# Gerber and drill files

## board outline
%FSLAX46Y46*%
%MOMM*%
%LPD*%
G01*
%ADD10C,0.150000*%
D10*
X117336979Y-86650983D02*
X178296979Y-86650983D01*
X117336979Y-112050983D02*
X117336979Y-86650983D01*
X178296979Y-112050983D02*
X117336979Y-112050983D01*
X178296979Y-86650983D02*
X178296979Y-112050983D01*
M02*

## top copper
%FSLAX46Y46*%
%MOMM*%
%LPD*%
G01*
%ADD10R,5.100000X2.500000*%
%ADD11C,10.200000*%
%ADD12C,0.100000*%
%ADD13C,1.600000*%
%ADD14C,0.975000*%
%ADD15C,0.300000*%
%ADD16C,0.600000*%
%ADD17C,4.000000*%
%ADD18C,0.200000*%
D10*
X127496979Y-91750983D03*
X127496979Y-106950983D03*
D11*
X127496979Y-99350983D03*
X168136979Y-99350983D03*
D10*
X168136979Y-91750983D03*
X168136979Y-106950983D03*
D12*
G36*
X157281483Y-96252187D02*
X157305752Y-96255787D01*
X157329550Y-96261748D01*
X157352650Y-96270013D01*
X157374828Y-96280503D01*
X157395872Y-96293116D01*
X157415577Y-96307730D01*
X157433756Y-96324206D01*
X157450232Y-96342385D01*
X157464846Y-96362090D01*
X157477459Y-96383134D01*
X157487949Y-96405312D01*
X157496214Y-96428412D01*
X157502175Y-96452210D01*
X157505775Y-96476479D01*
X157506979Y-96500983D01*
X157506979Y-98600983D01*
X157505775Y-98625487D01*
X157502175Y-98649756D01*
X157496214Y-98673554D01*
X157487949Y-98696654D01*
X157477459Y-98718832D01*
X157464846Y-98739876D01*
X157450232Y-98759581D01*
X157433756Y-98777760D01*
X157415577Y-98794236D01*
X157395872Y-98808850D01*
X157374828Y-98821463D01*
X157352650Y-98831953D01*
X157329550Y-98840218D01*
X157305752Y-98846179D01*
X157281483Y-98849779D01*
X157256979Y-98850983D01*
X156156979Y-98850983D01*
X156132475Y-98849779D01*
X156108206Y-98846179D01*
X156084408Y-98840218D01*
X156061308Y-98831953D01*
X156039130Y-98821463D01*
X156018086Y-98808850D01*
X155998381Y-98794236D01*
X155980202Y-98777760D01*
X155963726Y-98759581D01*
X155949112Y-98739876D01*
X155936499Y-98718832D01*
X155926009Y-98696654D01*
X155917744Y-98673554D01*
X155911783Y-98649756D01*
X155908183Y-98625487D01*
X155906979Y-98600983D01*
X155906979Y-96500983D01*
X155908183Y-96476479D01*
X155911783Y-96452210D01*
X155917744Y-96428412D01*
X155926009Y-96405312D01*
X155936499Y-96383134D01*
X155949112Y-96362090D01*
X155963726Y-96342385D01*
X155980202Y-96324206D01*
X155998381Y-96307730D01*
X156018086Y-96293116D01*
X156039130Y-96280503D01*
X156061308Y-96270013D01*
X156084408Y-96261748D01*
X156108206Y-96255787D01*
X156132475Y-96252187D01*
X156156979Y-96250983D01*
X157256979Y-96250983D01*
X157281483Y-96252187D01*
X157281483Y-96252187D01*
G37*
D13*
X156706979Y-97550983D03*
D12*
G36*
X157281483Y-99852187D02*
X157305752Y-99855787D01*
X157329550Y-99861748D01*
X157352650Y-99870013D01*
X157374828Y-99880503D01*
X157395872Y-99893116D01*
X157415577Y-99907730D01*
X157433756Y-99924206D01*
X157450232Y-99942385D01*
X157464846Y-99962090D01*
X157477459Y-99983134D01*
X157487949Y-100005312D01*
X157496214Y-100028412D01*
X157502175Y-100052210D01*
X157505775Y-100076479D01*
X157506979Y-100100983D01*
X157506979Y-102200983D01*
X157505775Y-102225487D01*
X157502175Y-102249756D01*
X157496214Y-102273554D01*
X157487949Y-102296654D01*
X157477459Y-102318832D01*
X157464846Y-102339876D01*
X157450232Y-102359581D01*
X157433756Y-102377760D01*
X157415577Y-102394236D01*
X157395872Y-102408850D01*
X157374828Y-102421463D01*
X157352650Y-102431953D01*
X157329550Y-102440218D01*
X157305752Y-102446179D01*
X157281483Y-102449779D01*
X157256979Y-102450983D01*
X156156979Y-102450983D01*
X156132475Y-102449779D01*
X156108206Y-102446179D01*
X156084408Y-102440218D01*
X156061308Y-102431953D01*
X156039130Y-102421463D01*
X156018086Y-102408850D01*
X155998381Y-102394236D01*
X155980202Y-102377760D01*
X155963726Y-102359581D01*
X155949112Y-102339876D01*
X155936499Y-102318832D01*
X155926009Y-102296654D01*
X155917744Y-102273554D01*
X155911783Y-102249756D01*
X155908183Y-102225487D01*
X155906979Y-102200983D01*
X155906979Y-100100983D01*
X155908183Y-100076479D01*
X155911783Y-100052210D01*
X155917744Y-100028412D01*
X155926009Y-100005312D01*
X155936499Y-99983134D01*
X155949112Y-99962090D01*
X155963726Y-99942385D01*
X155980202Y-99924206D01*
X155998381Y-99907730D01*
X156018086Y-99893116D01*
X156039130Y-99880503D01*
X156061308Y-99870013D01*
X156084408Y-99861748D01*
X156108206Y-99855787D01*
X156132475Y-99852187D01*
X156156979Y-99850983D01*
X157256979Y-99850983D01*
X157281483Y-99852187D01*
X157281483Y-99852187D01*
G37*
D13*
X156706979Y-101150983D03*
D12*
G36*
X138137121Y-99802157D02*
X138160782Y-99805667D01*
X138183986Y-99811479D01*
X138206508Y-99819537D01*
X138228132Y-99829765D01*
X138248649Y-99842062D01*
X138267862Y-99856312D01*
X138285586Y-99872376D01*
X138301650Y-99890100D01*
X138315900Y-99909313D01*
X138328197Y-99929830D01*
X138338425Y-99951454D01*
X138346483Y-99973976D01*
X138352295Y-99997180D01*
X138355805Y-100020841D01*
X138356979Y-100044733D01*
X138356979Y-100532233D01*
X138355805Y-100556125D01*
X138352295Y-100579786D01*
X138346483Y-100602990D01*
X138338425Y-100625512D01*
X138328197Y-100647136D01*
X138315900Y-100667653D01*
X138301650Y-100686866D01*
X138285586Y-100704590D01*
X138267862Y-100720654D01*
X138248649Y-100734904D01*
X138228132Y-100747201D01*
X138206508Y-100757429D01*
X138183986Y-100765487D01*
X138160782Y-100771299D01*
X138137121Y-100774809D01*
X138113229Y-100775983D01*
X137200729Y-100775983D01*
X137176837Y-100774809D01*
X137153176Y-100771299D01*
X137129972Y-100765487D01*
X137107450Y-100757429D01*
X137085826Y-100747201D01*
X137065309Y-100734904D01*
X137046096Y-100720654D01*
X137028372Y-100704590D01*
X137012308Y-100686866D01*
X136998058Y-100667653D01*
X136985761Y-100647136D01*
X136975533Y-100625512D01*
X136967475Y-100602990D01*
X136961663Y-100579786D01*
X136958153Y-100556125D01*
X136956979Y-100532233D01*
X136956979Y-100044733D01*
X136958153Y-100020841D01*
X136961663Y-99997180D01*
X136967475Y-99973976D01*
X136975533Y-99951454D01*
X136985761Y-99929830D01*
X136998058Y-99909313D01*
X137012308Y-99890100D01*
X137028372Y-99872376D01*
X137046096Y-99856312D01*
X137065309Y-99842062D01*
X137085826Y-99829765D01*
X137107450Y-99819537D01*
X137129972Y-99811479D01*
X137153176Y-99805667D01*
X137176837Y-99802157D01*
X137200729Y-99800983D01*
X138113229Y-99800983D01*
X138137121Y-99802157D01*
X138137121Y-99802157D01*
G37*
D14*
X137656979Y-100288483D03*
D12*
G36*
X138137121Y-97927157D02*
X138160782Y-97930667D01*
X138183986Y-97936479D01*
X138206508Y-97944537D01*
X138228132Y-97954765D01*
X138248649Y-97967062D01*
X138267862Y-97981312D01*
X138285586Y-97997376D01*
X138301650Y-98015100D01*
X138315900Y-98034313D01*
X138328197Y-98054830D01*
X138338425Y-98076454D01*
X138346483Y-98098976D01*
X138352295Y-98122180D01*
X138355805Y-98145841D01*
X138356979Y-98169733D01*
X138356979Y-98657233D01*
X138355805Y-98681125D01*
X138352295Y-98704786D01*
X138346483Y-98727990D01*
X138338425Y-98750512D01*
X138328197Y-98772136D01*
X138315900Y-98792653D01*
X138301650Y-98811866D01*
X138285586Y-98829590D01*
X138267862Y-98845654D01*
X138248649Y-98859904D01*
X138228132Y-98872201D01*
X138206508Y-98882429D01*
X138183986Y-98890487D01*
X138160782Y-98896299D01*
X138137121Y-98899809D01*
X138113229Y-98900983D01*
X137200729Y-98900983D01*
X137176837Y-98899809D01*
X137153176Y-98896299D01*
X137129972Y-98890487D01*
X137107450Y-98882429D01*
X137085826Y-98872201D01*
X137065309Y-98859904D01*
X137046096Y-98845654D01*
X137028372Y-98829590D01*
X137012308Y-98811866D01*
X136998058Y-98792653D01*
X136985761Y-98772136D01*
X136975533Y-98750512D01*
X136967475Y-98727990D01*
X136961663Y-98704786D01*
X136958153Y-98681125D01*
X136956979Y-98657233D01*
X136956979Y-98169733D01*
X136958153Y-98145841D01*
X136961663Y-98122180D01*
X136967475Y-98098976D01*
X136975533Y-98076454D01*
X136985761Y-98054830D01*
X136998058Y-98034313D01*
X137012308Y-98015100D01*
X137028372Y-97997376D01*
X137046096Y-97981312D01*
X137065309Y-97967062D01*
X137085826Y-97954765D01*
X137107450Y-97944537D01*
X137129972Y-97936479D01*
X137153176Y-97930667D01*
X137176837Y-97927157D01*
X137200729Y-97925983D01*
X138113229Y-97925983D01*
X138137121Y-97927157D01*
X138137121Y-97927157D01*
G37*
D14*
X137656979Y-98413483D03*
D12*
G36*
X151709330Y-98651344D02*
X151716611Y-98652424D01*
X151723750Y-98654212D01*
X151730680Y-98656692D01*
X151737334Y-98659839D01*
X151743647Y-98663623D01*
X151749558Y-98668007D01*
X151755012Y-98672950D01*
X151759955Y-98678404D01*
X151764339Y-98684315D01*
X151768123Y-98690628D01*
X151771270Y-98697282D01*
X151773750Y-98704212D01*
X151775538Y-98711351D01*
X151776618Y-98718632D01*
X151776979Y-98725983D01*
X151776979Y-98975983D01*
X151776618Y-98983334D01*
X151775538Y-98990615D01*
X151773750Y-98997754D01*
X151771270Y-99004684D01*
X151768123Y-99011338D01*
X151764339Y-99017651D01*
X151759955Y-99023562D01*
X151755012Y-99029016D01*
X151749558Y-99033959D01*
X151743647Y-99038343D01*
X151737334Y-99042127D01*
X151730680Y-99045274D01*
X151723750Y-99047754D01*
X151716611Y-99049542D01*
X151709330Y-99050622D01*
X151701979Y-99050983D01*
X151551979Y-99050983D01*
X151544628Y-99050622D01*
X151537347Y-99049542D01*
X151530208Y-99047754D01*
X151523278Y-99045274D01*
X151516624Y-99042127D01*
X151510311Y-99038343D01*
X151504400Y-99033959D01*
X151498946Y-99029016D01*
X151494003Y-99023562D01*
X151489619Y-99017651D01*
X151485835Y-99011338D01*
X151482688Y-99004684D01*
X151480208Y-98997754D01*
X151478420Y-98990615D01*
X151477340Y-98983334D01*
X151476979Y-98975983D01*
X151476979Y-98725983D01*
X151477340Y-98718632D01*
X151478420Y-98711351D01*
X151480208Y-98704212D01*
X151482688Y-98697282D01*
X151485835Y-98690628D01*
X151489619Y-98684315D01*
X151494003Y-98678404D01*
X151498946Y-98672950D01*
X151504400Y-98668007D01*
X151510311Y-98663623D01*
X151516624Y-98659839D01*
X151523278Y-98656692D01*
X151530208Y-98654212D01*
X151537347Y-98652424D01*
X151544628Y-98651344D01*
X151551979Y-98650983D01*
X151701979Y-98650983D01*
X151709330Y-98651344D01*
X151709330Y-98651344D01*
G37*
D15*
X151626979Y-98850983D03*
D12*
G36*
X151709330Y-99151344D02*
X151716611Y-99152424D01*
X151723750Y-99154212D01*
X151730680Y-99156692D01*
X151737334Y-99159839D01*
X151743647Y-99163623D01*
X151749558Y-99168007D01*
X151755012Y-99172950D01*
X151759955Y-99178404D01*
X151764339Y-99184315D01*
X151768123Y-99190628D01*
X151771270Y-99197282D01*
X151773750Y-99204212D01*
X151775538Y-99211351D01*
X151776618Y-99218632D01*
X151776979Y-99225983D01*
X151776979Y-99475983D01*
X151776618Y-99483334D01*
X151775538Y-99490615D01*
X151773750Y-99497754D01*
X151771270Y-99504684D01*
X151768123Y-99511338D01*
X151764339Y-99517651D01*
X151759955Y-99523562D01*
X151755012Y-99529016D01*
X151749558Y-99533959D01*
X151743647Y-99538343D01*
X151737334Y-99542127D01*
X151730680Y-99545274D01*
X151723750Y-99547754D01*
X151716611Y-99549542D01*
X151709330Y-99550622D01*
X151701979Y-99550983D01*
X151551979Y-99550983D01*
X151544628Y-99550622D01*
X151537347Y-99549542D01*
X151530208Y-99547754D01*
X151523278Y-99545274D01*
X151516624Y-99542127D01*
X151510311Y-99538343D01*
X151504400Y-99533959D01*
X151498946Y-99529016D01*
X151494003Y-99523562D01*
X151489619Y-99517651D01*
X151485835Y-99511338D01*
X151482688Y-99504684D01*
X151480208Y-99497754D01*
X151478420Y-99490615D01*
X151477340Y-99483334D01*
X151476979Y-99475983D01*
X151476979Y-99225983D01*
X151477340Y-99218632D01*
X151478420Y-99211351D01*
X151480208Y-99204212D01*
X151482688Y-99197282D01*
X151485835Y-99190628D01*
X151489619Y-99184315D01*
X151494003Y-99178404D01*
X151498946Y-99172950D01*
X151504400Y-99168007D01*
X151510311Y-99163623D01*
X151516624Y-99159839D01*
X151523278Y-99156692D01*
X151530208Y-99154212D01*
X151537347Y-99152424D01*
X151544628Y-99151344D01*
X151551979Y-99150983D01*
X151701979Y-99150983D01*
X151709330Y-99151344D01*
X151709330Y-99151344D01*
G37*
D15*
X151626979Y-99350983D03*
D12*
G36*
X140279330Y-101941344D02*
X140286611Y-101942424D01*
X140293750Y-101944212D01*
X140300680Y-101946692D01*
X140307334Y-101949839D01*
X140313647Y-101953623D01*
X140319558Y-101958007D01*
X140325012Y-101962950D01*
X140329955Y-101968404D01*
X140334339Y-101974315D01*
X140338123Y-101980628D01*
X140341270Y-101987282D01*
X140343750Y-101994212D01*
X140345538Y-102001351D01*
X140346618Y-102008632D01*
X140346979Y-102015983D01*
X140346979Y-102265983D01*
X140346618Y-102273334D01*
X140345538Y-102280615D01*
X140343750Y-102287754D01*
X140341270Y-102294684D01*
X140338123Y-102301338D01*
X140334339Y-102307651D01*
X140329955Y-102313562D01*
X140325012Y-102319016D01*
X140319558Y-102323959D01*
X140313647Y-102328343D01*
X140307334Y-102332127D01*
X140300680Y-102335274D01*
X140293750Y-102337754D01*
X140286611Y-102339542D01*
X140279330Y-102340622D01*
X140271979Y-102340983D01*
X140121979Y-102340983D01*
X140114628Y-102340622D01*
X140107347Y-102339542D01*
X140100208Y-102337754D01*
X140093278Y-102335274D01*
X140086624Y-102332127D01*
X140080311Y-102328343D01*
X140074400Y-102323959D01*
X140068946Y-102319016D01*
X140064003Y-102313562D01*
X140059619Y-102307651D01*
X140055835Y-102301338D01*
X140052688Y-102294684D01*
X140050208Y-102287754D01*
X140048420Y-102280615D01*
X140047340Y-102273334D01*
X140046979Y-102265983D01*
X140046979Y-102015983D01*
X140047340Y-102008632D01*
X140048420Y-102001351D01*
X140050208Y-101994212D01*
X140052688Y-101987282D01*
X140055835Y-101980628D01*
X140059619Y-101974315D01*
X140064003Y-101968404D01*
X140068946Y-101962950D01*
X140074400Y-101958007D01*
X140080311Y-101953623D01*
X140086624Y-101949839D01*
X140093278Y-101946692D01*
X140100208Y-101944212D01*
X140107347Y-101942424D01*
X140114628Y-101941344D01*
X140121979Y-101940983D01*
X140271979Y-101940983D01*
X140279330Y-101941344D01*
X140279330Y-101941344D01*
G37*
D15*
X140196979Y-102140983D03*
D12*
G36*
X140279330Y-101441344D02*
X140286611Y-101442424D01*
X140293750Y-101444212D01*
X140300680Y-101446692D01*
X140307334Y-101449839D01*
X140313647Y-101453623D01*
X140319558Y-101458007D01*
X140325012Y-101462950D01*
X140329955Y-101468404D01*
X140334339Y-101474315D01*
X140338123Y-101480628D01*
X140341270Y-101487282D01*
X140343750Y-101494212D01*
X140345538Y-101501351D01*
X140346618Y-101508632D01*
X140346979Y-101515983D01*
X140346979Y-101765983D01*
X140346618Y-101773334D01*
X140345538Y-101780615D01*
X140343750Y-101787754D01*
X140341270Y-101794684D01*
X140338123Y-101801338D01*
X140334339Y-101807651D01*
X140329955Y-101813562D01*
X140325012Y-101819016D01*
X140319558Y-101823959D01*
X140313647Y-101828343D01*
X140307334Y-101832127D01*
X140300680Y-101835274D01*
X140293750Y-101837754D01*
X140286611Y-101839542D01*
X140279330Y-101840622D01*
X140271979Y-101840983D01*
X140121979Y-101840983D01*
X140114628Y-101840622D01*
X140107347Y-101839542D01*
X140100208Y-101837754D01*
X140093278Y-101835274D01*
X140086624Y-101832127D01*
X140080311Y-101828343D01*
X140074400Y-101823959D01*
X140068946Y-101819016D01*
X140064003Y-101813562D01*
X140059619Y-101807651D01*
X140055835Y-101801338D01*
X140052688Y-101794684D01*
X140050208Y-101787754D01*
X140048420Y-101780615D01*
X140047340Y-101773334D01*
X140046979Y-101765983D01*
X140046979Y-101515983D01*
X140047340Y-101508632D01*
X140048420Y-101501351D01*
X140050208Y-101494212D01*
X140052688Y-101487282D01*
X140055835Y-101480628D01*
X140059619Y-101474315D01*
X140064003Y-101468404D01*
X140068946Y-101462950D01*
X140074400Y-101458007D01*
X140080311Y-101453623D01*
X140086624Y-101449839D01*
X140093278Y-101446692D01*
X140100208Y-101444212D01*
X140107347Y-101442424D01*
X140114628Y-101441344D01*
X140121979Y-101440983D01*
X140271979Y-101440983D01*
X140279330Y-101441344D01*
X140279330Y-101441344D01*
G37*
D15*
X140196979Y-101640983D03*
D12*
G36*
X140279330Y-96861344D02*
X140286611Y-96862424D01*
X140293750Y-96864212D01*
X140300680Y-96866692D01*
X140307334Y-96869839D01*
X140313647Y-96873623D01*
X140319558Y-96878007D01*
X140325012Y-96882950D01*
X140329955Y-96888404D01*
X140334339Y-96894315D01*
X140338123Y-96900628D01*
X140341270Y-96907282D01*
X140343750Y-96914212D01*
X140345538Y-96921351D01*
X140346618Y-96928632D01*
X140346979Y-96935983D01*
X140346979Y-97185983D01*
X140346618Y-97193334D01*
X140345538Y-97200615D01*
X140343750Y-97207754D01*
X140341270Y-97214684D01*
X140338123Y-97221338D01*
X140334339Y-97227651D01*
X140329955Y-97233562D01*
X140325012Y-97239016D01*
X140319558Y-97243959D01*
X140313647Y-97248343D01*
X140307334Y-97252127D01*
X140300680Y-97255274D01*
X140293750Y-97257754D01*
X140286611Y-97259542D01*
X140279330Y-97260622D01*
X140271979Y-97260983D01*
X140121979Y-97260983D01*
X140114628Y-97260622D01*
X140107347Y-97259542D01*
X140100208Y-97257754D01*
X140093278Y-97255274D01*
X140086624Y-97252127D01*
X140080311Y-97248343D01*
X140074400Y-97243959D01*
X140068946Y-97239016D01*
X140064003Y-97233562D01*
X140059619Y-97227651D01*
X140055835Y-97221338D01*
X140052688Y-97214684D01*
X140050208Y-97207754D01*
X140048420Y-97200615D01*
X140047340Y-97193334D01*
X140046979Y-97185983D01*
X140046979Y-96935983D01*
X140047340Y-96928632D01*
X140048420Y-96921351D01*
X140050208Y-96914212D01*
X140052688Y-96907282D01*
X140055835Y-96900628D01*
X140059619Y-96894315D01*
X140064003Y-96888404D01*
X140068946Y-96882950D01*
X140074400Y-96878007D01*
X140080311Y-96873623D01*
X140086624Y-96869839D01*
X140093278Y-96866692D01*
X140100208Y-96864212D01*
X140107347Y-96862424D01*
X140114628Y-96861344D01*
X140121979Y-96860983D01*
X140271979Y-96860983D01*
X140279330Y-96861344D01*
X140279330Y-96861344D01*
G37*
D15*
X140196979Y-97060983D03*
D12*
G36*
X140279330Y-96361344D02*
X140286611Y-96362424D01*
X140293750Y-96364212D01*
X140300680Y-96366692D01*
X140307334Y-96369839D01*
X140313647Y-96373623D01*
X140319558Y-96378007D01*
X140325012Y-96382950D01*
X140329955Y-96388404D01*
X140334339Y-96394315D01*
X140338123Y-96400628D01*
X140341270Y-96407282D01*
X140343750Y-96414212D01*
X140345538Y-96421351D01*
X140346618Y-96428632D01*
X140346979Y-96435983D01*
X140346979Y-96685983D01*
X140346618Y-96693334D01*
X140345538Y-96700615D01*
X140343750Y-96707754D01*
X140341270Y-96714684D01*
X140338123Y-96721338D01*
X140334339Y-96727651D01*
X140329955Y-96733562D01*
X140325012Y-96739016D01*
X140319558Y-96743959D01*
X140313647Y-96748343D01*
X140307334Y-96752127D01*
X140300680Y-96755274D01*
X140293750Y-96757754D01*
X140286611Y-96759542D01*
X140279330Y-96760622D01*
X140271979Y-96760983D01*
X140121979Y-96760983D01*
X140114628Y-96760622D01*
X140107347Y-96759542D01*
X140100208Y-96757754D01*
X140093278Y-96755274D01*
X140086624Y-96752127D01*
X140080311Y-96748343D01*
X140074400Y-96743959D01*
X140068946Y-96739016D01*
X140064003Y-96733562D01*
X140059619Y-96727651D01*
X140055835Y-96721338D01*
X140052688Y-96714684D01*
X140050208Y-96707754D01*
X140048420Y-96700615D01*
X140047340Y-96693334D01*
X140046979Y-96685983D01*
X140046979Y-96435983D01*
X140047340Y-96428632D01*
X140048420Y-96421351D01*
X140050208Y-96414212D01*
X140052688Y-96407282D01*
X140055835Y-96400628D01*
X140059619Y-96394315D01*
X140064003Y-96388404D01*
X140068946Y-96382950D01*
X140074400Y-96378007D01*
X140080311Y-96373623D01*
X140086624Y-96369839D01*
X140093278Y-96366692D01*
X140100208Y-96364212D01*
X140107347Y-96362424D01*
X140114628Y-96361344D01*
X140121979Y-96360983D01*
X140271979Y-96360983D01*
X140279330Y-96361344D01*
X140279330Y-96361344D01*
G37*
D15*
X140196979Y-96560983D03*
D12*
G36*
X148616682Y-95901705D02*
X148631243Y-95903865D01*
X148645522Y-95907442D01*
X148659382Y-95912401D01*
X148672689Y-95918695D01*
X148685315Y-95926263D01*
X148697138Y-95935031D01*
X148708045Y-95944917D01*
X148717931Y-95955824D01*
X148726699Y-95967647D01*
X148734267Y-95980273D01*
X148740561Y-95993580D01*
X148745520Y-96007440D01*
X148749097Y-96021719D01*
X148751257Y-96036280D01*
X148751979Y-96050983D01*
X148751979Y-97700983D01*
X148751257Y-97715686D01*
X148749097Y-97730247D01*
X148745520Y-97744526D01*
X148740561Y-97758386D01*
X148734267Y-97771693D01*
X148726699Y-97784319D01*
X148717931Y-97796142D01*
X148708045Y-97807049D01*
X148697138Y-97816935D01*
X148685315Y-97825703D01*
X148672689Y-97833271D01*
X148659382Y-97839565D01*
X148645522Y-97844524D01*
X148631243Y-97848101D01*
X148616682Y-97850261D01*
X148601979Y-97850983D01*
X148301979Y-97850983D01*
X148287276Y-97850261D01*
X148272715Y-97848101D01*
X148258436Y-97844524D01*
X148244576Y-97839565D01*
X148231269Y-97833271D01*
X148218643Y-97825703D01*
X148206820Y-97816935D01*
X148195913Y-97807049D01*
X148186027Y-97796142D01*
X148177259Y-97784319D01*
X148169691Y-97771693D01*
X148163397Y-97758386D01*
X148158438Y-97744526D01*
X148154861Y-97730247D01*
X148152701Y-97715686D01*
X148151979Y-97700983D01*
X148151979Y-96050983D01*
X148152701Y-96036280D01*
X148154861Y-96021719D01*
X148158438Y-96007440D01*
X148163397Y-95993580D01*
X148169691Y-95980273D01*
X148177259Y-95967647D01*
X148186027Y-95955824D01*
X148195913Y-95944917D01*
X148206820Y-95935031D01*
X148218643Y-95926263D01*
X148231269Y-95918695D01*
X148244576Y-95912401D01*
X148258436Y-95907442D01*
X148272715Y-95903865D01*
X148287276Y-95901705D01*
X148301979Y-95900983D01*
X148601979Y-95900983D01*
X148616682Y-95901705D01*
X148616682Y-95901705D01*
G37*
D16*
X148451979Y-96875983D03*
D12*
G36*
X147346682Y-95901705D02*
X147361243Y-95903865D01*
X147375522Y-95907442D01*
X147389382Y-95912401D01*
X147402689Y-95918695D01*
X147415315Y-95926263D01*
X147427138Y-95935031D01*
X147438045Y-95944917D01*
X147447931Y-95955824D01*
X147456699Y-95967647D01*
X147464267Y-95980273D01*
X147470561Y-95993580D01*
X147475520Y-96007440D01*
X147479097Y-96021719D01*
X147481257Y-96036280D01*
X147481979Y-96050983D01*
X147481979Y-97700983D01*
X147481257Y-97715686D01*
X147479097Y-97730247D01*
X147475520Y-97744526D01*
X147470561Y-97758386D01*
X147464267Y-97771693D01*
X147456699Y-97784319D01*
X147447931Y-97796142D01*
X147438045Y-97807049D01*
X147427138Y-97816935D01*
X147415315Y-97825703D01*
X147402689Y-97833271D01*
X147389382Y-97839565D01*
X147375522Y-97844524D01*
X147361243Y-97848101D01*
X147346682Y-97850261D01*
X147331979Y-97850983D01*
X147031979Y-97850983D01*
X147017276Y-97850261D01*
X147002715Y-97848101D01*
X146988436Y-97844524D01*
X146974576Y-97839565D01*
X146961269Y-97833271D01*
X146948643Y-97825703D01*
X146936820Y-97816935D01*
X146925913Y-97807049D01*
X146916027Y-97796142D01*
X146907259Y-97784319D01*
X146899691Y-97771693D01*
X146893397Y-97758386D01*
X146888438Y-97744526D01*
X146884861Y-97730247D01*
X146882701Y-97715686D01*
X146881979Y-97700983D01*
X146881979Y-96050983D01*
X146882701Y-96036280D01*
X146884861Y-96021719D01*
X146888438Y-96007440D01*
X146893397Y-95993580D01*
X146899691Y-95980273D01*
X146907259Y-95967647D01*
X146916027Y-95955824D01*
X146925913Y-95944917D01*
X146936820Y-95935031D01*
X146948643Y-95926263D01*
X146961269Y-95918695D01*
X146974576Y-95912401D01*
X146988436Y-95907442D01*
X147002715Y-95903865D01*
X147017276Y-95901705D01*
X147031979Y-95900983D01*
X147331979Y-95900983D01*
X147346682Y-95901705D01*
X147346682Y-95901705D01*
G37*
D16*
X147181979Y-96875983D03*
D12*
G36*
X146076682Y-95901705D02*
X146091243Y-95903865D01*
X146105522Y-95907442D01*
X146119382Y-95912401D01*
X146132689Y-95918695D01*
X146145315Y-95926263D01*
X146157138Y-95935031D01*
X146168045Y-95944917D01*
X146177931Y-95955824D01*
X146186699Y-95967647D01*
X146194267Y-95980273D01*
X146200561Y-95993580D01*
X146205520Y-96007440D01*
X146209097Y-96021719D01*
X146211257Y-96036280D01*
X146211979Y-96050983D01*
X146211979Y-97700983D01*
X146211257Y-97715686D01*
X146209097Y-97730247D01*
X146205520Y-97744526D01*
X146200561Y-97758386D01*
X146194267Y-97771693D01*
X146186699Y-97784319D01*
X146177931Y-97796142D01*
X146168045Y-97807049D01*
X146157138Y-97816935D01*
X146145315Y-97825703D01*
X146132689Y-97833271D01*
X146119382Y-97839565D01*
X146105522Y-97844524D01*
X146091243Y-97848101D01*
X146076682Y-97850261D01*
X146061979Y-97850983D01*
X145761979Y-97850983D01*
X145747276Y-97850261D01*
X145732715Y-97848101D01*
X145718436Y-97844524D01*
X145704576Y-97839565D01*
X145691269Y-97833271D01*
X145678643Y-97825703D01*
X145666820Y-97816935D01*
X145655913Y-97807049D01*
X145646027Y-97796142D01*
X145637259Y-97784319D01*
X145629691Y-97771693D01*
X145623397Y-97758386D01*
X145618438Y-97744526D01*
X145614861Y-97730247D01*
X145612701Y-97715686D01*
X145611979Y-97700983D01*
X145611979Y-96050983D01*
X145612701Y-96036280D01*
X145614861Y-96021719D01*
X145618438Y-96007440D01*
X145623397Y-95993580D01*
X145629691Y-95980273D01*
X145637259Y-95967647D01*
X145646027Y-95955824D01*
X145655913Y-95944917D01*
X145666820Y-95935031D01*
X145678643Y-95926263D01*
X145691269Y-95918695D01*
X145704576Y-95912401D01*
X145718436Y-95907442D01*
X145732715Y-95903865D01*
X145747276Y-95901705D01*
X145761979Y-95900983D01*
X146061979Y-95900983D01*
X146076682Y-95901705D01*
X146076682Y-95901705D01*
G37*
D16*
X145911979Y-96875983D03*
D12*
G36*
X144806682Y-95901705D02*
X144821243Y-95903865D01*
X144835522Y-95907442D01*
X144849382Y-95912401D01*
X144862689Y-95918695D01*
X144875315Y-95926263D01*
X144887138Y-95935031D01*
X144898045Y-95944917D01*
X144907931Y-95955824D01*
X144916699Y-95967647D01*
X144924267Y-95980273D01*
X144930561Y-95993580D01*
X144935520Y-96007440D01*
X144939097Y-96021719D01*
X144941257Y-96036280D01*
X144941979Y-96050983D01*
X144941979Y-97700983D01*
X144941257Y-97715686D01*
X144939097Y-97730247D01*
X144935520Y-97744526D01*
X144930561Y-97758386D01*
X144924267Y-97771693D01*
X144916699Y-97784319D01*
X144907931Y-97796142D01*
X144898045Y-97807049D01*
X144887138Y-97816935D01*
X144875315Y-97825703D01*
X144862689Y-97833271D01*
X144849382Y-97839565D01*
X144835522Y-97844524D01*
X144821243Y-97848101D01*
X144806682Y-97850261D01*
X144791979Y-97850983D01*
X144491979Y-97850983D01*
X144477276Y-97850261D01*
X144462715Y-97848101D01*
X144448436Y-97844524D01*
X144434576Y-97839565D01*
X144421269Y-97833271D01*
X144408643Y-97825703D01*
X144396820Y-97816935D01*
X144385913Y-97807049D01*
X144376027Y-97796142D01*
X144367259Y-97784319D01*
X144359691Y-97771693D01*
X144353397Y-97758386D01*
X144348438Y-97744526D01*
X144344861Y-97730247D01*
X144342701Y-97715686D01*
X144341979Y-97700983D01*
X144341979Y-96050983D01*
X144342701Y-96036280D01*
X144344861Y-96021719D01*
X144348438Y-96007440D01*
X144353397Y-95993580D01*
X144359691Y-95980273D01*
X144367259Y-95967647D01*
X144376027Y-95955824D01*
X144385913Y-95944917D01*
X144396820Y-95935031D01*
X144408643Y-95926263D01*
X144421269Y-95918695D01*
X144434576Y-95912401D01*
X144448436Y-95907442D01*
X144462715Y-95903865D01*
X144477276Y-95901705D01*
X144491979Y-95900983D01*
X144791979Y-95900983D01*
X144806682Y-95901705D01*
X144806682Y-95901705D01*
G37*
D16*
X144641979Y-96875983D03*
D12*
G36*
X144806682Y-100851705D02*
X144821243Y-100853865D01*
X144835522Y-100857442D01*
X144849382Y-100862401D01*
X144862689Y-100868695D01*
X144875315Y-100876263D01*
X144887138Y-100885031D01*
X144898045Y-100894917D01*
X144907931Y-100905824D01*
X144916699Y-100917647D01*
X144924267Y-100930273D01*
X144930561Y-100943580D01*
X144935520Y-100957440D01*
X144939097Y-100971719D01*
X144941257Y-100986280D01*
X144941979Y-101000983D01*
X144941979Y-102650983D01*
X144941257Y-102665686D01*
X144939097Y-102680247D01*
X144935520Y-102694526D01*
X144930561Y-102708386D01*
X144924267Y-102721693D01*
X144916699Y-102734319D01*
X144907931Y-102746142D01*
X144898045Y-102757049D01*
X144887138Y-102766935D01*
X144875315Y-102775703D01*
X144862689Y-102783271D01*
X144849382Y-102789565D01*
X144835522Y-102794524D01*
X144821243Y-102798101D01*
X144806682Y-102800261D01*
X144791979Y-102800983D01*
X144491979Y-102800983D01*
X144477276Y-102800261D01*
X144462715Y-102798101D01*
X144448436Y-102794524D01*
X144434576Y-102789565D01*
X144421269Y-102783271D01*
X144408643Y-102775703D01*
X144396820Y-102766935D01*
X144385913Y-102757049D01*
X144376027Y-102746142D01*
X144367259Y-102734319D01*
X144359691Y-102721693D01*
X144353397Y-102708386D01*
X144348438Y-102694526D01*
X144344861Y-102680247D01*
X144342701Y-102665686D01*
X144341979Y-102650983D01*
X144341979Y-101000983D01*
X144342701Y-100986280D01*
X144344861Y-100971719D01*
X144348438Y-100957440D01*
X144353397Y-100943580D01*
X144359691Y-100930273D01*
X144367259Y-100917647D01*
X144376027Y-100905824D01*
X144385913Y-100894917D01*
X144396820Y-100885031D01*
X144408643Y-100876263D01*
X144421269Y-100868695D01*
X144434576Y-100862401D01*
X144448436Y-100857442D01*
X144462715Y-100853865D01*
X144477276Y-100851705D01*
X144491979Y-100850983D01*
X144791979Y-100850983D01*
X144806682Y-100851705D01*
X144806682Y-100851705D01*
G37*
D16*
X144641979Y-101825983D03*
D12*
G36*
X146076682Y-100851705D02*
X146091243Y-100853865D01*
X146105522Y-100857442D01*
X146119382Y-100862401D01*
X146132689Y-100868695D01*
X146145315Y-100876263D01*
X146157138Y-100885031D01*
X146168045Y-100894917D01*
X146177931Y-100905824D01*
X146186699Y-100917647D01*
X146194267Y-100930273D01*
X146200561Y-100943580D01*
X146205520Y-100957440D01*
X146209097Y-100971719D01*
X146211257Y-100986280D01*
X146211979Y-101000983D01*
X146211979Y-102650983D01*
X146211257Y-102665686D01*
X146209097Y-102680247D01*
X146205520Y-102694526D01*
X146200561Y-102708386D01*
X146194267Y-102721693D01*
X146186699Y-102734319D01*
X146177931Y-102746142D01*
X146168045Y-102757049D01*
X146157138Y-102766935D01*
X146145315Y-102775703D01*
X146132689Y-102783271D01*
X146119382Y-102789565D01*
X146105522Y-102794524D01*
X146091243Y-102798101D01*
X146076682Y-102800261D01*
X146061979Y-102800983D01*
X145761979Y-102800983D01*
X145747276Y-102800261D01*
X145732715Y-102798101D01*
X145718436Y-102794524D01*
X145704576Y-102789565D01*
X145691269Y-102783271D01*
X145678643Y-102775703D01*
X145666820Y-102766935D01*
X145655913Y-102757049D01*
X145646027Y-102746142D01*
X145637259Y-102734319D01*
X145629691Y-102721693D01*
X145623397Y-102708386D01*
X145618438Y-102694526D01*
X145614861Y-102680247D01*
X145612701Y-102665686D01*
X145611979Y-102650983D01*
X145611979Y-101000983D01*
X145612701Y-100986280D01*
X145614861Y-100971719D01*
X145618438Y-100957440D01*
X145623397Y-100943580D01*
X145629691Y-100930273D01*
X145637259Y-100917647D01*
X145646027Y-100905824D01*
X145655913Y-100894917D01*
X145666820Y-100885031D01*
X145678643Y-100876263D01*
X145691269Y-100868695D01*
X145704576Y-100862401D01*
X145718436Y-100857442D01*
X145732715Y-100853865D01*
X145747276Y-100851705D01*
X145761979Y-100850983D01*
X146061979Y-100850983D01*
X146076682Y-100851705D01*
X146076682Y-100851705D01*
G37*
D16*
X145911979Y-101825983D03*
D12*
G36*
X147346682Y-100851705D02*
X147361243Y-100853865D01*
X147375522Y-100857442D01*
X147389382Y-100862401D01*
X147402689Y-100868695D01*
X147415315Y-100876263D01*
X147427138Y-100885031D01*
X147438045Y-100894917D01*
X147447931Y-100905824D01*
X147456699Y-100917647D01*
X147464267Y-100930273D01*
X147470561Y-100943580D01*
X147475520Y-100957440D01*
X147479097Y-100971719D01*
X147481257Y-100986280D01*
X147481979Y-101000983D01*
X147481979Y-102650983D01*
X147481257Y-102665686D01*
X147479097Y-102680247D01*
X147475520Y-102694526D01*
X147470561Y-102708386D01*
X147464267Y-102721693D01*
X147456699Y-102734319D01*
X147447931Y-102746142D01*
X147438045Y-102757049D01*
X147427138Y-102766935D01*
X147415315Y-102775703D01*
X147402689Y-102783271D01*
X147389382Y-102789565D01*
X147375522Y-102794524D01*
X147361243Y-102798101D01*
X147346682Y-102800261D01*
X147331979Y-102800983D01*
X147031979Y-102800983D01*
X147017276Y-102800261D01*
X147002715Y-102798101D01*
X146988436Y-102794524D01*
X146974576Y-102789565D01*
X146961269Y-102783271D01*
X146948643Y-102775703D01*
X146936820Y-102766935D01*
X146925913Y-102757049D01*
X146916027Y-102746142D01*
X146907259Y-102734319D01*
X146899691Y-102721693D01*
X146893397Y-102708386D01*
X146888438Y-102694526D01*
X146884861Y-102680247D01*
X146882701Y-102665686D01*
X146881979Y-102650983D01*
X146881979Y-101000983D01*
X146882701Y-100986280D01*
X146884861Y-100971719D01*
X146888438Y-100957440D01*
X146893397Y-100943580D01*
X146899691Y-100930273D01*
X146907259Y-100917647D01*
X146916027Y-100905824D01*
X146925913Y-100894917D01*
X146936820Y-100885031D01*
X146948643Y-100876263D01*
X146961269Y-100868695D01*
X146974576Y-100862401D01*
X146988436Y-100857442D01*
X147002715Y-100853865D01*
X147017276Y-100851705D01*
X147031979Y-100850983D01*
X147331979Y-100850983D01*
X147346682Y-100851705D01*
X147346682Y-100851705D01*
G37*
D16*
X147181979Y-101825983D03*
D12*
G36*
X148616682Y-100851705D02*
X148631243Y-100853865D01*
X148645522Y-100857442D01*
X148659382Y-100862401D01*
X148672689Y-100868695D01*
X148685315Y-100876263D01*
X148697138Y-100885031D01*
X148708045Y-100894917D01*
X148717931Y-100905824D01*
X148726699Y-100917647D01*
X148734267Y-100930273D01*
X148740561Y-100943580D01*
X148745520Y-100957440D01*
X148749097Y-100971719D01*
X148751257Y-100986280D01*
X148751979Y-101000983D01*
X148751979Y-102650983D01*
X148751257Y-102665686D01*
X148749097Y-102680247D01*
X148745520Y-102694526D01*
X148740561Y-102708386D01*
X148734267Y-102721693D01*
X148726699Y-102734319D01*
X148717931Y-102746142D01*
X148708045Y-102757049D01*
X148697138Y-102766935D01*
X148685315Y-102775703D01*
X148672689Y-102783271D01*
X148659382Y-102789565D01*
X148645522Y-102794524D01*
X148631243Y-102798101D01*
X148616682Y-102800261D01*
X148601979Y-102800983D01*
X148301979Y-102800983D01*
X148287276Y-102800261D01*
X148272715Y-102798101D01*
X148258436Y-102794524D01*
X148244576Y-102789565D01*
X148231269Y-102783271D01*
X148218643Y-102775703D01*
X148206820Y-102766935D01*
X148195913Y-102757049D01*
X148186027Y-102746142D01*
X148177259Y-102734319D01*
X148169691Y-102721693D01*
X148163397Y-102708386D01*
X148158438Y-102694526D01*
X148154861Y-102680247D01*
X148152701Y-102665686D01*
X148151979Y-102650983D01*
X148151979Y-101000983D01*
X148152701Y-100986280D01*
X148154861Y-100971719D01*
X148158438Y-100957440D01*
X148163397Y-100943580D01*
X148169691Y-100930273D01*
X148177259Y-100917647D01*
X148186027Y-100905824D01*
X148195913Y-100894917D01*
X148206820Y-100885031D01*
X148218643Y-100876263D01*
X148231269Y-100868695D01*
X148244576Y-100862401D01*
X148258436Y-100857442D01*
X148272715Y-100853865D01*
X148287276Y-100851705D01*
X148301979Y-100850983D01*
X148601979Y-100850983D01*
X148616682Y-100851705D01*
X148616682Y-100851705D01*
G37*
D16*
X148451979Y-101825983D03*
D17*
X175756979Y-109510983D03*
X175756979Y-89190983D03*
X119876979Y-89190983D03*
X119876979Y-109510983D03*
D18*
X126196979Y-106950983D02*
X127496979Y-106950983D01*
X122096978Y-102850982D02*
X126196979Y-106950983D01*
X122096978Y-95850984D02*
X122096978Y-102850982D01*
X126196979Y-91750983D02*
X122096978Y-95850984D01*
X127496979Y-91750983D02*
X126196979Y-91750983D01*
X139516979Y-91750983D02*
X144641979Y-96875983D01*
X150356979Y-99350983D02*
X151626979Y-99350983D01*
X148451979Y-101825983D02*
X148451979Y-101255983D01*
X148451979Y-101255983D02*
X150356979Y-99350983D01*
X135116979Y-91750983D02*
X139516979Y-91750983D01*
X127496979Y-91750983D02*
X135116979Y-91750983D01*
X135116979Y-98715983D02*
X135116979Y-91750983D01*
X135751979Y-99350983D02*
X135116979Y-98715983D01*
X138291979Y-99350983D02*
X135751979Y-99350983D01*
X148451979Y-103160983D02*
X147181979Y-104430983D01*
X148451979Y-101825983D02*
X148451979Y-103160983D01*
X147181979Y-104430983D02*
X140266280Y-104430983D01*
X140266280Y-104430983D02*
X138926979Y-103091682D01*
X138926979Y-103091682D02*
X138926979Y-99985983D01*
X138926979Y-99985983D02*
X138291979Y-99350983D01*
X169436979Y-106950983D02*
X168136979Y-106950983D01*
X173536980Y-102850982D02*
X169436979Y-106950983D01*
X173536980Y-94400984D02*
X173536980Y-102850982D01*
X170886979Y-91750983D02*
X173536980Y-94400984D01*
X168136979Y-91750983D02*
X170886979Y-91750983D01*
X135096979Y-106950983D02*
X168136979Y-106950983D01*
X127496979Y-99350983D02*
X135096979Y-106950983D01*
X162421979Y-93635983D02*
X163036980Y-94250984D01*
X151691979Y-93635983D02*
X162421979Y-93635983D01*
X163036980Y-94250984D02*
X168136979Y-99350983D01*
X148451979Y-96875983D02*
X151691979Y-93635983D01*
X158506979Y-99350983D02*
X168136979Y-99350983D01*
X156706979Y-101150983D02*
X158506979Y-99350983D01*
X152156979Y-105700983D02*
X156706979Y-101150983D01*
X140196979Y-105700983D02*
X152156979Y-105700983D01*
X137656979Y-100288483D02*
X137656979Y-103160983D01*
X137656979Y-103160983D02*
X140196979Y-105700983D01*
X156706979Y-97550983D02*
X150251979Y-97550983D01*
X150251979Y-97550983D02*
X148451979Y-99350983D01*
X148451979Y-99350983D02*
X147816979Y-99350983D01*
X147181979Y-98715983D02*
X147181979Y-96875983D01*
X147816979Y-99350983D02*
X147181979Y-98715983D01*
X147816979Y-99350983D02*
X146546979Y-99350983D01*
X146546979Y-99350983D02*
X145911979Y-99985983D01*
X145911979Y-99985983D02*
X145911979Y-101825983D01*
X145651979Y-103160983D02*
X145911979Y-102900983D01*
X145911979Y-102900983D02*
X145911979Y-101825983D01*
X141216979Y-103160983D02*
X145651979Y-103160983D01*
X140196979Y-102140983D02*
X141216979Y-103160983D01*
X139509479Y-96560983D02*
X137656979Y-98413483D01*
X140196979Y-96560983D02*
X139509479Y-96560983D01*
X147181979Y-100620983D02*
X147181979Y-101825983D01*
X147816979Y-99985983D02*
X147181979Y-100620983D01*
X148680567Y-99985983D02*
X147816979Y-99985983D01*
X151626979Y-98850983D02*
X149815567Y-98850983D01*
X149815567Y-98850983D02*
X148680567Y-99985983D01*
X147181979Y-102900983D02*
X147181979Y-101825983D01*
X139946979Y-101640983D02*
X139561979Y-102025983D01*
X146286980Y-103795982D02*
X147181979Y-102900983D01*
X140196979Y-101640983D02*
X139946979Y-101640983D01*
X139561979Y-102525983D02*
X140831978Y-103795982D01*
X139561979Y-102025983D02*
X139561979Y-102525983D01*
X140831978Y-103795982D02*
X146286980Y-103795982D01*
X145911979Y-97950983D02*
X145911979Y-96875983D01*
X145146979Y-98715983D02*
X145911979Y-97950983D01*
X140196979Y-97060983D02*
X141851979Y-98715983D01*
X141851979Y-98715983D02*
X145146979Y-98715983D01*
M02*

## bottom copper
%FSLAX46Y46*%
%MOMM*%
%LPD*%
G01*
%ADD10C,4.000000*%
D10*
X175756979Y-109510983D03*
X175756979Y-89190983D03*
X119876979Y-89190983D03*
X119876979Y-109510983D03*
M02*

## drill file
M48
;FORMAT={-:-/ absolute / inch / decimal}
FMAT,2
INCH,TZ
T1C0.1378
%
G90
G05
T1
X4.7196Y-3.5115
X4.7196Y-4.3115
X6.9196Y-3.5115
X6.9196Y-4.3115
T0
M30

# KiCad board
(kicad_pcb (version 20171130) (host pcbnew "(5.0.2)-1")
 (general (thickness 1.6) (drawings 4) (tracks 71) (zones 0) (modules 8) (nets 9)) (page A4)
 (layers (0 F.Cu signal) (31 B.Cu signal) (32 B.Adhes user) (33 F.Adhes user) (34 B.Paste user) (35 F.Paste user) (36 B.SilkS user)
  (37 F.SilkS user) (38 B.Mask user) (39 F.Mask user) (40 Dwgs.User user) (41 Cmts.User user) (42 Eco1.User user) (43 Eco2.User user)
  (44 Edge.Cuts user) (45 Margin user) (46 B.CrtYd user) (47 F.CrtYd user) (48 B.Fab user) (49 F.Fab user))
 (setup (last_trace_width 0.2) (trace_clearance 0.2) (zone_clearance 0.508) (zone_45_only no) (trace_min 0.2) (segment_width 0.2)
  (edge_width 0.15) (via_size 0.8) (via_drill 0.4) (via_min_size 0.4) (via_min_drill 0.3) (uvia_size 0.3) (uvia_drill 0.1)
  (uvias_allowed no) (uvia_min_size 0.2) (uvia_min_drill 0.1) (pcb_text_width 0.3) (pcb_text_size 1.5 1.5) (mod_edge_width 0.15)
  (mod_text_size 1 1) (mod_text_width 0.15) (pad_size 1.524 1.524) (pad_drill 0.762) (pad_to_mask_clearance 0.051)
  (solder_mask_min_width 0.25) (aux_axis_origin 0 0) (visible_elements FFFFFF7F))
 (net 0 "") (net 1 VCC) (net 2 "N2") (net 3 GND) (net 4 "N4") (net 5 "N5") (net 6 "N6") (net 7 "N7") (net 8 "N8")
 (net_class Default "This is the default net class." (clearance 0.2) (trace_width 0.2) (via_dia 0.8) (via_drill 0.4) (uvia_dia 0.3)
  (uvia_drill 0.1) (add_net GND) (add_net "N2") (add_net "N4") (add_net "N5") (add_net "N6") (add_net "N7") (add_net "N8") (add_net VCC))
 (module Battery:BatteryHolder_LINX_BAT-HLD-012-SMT (layer F.Cu) (at 127.496979 99.350983 270)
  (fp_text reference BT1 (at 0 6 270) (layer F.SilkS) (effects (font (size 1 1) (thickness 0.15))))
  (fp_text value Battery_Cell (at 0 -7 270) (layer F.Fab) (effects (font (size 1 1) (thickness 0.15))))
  (pad 1 smd rect (at -7.6 0 270) (size 2.5 5.1) (layers F.Cu F.Paste F.Mask) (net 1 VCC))
  (pad 1 smd rect (at 7.6 0 270) (size 2.5 5.1) (layers F.Cu F.Paste F.Mask) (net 1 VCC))
  (pad 2 smd circle (at 0 0 270) (size 10.2 10.2) (layers F.Cu F.Mask) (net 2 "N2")))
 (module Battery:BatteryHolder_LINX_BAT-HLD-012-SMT (layer F.Cu) (at 168.136979 99.350983 90)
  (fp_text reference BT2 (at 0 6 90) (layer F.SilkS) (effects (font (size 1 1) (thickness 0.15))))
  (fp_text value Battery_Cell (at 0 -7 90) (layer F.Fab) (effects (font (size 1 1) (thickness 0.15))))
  (pad 2 smd circle (at 0 0 90) (size 10.2 10.2) (layers F.Cu F.Mask) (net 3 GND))
  (pad 1 smd rect (at 7.6 0 90) (size 2.5 5.1) (layers F.Cu F.Paste F.Mask) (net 2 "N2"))
  (pad 1 smd rect (at -7.6 0 90) (size 2.5 5.1) (layers F.Cu F.Paste F.Mask) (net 2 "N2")))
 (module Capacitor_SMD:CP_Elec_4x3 (layer F.Cu) (at 156.706979 99.350983 270)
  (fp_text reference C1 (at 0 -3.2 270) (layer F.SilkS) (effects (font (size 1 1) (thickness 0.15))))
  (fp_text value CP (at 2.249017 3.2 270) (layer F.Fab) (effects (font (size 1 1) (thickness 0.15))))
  (pad 1 smd roundrect (at -1.8 0 270) (size 2.6 1.6) (layers F.Cu F.Paste F.Mask) (roundrect_rratio 0.15625) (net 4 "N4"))
  (pad 2 smd roundrect (at 1.8 0 270) (size 2.6 1.6) (layers F.Cu F.Paste F.Mask) (roundrect_rratio 0.15625) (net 3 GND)))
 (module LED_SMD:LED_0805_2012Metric (layer F.Cu) (at 137.656979 99.350983 90)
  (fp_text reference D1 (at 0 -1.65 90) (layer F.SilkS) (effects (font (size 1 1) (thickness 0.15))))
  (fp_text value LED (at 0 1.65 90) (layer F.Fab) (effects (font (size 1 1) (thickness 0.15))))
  (pad 1 smd roundrect (at -0.9375 0 90) (size 0.975 1.4) (layers F.Cu F.Paste F.Mask) (roundrect_rratio 0.25) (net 3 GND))
  (pad 2 smd roundrect (at 0.9375 0 90) (size 0.975 1.4) (layers F.Cu F.Paste F.Mask) (roundrect_rratio 0.25) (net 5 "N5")))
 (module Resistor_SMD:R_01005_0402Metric (layer F.Cu) (at 151.626979 99.100983 90)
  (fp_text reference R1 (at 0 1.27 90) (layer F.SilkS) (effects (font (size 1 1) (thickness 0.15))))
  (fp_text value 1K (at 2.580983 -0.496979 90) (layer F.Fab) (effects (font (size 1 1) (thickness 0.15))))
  (pad 2 smd roundrect (at 0.25 0 90) (size 0.4 0.3) (layers F.Cu F.Mask) (roundrect_rratio 0.25) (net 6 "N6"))
  (pad 1 smd roundrect (at -0.25 0 90) (size 0.4 0.3) (layers F.Cu F.Mask) (roundrect_rratio 0.25) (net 1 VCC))
  (pad "" smd roundrect (at 0.275 0 90) (size 0.27 0.27) (layers F.Paste) (roundrect_rratio 0.25))
  (pad "" smd roundrect (at -0.275 0 90) (size 0.27 0.27) (layers F.Paste) (roundrect_rratio 0.25)))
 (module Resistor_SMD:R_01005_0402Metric (layer F.Cu) (at 140.196979 101.890983 270)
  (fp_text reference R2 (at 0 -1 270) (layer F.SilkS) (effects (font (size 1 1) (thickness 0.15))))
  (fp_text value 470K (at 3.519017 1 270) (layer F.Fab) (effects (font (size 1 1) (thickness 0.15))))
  (pad 2 smd roundrect (at 0.25 0 270) (size 0.4 0.3) (layers F.Cu F.Mask) (roundrect_rratio 0.25) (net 4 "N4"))
  (pad 1 smd roundrect (at -0.25 0 270) (size 0.4 0.3) (layers F.Cu F.Mask) (roundrect_rratio 0.25) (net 6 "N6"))
  (pad "" smd roundrect (at 0.275 0 270) (size 0.27 0.27) (layers F.Paste) (roundrect_rratio 0.25))
  (pad "" smd roundrect (at -0.275 0 270) (size 0.27 0.27) (layers F.Paste) (roundrect_rratio 0.25)))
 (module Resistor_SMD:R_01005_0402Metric (layer F.Cu) (at 140.196979 96.810983 270)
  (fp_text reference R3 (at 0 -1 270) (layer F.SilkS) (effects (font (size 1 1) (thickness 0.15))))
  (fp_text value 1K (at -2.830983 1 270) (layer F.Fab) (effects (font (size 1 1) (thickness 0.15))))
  (pad 2 smd roundrect (at 0.25 0 270) (size 0.4 0.3) (layers F.Cu F.Mask) (roundrect_rratio 0.25) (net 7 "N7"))
  (pad 1 smd roundrect (at -0.25 0 270) (size 0.4 0.3) (layers F.Cu F.Mask) (roundrect_rratio 0.25) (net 5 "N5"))
  (pad "" smd roundrect (at 0.275 0 270) (size 0.27 0.27) (layers F.Paste) (roundrect_rratio 0.25))
  (pad "" smd roundrect (at -0.275 0 270) (size 0.27 0.27) (layers F.Paste) (roundrect_rratio 0.25)))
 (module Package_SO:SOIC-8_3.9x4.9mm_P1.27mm (layer F.Cu) (at 146.546979 99.350983 270)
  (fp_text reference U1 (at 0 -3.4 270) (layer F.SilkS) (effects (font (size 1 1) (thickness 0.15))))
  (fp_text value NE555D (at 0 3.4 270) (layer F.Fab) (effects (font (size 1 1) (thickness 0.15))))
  (pad 1 smd roundrect (at -2.475 -1.905 270) (size 1.95 0.6) (layers F.Cu F.Paste F.Mask) (roundrect_rratio 0.25) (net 3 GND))
  (pad 2 smd roundrect (at -2.475 -0.635 270) (size 1.95 0.6) (layers F.Cu F.Paste F.Mask) (roundrect_rratio 0.25) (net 4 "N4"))
  (pad 3 smd roundrect (at -2.475 0.635 270) (size 1.95 0.6) (layers F.Cu F.Paste F.Mask) (roundrect_rratio 0.25) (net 7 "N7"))
  (pad 4 smd roundrect (at -2.475 1.905 270) (size 1.95 0.6) (layers F.Cu F.Paste F.Mask) (roundrect_rratio 0.25) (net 1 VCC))
  (pad 5 smd roundrect (at 2.475 1.905 270) (size 1.95 0.6) (layers F.Cu F.Paste F.Mask) (roundrect_rratio 0.25) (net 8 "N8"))
  (pad 6 smd roundrect (at 2.475 0.635 270) (size 1.95 0.6) (layers F.Cu F.Paste F.Mask) (roundrect_rratio 0.25) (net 4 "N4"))
  (pad 7 smd roundrect (at 2.475 -0.635 270) (size 1.95 0.6) (layers F.Cu F.Paste F.Mask) (roundrect_rratio 0.25) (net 6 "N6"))
  (pad 8 smd roundrect (at 2.475 -1.905 270) (size 1.95 0.6) (layers F.Cu F.Paste F.Mask) (roundrect_rratio 0.25) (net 1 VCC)))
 (gr_line (start 117.336979 86.650983) (end 178.296979 86.650983) (layer Edge.Cuts) (width 0.15))
 (gr_line (start 117.336979 112.050983) (end 117.336979 86.650983) (layer Edge.Cuts) (width 0.15))
 (gr_line (start 178.296979 112.050983) (end 117.336979 112.050983) (layer Edge.Cuts) (width 0.15))
 (gr_line (start 178.296979 86.650983) (end 178.296979 112.050983) (layer Edge.Cuts) (width 0.15))
 (via (at 175.756979 109.510983) (size 4) (drill 3.5) (layers F.Cu B.Cu) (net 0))
 (via (at 175.756979 89.190983) (size 4) (drill 3.5) (layers F.Cu B.Cu) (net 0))
 (via (at 119.876979 89.190983) (size 4) (drill 3.5) (layers F.Cu B.Cu) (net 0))
 (via (at 119.876979 109.510983) (size 4) (drill 3.5) (layers F.Cu B.Cu) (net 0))
 (segment (start 126.196979 106.950983) (end 127.496979 106.950983) (width 0.2) (layer F.Cu) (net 1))
 (segment (start 122.096978 102.850982) (end 126.196979 106.950983) (width 0.2) (layer F.Cu) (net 1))
 (segment (start 122.096978 95.850984) (end 122.096978 102.850982) (width 0.2) (layer F.Cu) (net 1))
 (segment (start 126.196979 91.750983) (end 122.096978 95.850984) (width 0.2) (layer F.Cu) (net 1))
 (segment (start 127.496979 91.750983) (end 126.196979 91.750983) (width 0.2) (layer F.Cu) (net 1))
 (segment (start 139.516979 91.750983) (end 144.641979 96.875983) (width 0.2) (layer F.Cu) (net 1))
 (segment (start 150.356979 99.350983) (end 151.626979 99.350983) (width 0.2) (layer F.Cu) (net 1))
 (segment (start 148.451979 101.825983) (end 148.451979 101.255983) (width 0.2) (layer F.Cu) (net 1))
 (segment (start 148.451979 101.255983) (end 150.356979 99.350983) (width 0.2) (layer F.Cu) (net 1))
 (segment (start 135.116979 91.750983) (end 139.516979 91.750983) (width 0.2) (layer F.Cu) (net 1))
 (segment (start 127.496979 91.750983) (end 135.116979 91.750983) (width 0.2) (layer F.Cu) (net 1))
 (segment (start 135.116979 98.715983) (end 135.116979 91.750983) (width 0.2) (layer F.Cu) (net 1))
 (segment (start 135.751979 99.350983) (end 135.116979 98.715983) (width 0.2) (layer F.Cu) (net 1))
 (segment (start 138.291979 99.350983) (end 135.751979 99.350983) (width 0.2) (layer F.Cu) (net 1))
 (segment (start 148.451979 103.160983) (end 147.181979 104.430983) (width 0.2) (layer F.Cu) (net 1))
 (segment (start 148.451979 101.825983) (end 148.451979 103.160983) (width 0.2) (layer F.Cu) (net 1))
 (segment (start 147.181979 104.430983) (end 140.26628 104.430983) (width 0.2) (layer F.Cu) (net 1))
 (segment (start 140.26628 104.430983) (end 138.926979 103.091682) (width 0.2) (layer F.Cu) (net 1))
 (segment (start 138.926979 103.091682) (end 138.926979 99.985983) (width 0.2) (layer F.Cu) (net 1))
 (segment (start 138.926979 99.985983) (end 138.291979 99.350983) (width 0.2) (layer F.Cu) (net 1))
 (segment (start 169.436979 106.950983) (end 168.136979 106.950983) (width 0.2) (layer F.Cu) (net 2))
 (segment (start 173.53698 102.850982) (end 169.436979 106.950983) (width 0.2) (layer F.Cu) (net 2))
 (segment (start 173.53698 94.400984) (end 173.53698 102.850982) (width 0.2) (layer F.Cu) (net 2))
 (segment (start 170.886979 91.750983) (end 173.53698 94.400984) (width 0.2) (layer F.Cu) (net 2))
 (segment (start 168.136979 91.750983) (end 170.886979 91.750983) (width 0.2) (layer F.Cu) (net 2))
 (segment (start 135.096979 106.950983) (end 168.136979 106.950983) (width 0.2) (layer F.Cu) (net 2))
 (segment (start 127.496979 99.350983) (end 135.096979 106.950983) (width 0.2) (layer F.Cu) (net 2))
 (segment (start 162.421979 93.635983) (end 163.03698 94.250984) (width 0.2) (layer F.Cu) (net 3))
 (segment (start 151.691979 93.635983) (end 162.421979 93.635983) (width 0.2) (layer F.Cu) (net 3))
 (segment (start 163.03698 94.250984) (end 168.136979 99.350983) (width 0.2) (layer F.Cu) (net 3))
 (segment (start 148.451979 96.875983) (end 151.691979 93.635983) (width 0.2) (layer F.Cu) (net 3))
 (segment (start 158.506979 99.350983) (end 168.136979 99.350983) (width 0.2) (layer F.Cu) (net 3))
 (segment (start 156.706979 101.150983) (end 158.506979 99.350983) (width 0.2) (layer F.Cu) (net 3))
 (segment (start 152.156979 105.700983) (end 156.706979 101.150983) (width 0.2) (layer F.Cu) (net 3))
 (segment (start 140.196979 105.700983) (end 152.156979 105.700983) (width 0.2) (layer F.Cu) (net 3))
 (segment (start 137.656979 100.288483) (end 137.656979 103.160983) (width 0.2) (layer F.Cu) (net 3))
 (segment (start 137.656979 103.160983) (end 140.196979 105.700983) (width 0.2) (layer F.Cu) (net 3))
 (segment (start 156.706979 97.550983) (end 150.251979 97.550983) (width 0.2) (layer F.Cu) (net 4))
 (segment (start 150.251979 97.550983) (end 148.451979 99.350983) (width 0.2) (layer F.Cu) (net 4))
 (segment (start 148.451979 99.350983) (end 147.816979 99.350983) (width 0.2) (layer F.Cu) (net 4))
 (segment (start 147.181979 98.715983) (end 147.181979 96.875983) (width 0.2) (layer F.Cu) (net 4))
 (segment (start 147.816979 99.350983) (end 147.181979 98.715983) (width 0.2) (layer F.Cu) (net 4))
 (segment (start 147.816979 99.350983) (end 146.546979 99.350983) (width 0.2) (layer F.Cu) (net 4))
 (segment (start 146.546979 99.350983) (end 145.911979 99.985983) (width 0.2) (layer F.Cu) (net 4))
 (segment (start 145.911979 99.985983) (end 145.911979 101.825983) (width 0.2) (layer F.Cu) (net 4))
 (segment (start 145.651979 103.160983) (end 145.911979 102.900983) (width 0.2) (layer F.Cu) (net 4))
 (segment (start 145.911979 102.900983) (end 145.911979 101.825983) (width 0.2) (layer F.Cu) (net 4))
 (segment (start 141.216979 103.160983) (end 145.651979 103.160983) (width 0.2) (layer F.Cu) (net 4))
 (segment (start 140.196979 102.140983) (end 141.216979 103.160983) (width 0.2) (layer F.Cu) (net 4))
 (segment (start 139.509479 96.560983) (end 137.656979 98.413483) (width 0.2) (layer F.Cu) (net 5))
 (segment (start 140.196979 96.560983) (end 139.509479 96.560983) (width 0.2) (layer F.Cu) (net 5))
 (segment (start 147.181979 100.620983) (end 147.181979 101.825983) (width 0.2) (layer F.Cu) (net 6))
 (segment (start 147.816979 99.985983) (end 147.181979 100.620983) (width 0.2) (layer F.Cu) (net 6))
 (segment (start 148.680567 99.985983) (end 147.816979 99.985983) (width 0.2) (layer F.Cu) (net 6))
 (segment (start 151.626979 98.850983) (end 149.815567 98.850983) (width 0.2) (layer F.Cu) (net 6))
 (segment (start 149.815567 98.850983) (end 148.680567 99.985983) (width 0.2) (layer F.Cu) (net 6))
 (segment (start 147.181979 102.900983) (end 147.181979 101.825983) (width 0.2) (layer F.Cu) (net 6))
 (segment (start 139.946979 101.640983) (end 139.561979 102.025983) (width 0.2) (layer F.Cu) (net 6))
 (segment (start 146.28698 103.795982) (end 147.181979 102.900983) (width 0.2) (layer F.Cu) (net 6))
 (segment (start 140.196979 101.640983) (end 139.946979 101.640983) (width 0.2) (layer F.Cu) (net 6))
 (segment (start 139.561979 102.525983) (end 140.831978 103.795982) (width 0.2) (layer F.Cu) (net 6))
 (segment (start 139.561979 102.025983) (end 139.561979 102.525983) (width 0.2) (layer F.Cu) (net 6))
 (segment (start 140.831978 103.795982) (end 146.28698 103.795982) (width 0.2) (layer F.Cu) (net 6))
 (segment (start 145.911979 97.950983) (end 145.911979 96.875983) (width 0.2) (layer F.Cu) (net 7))
 (segment (start 145.146979 98.715983) (end 145.911979 97.950983) (width 0.2) (layer F.Cu) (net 7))
 (segment (start 140.196979 97.060983) (end 141.851979 98.715983) (width 0.2) (layer F.Cu) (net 7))
 (segment (start 141.851979 98.715983) (end 145.146979 98.715983) (width 0.2) (layer F.Cu) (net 7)))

